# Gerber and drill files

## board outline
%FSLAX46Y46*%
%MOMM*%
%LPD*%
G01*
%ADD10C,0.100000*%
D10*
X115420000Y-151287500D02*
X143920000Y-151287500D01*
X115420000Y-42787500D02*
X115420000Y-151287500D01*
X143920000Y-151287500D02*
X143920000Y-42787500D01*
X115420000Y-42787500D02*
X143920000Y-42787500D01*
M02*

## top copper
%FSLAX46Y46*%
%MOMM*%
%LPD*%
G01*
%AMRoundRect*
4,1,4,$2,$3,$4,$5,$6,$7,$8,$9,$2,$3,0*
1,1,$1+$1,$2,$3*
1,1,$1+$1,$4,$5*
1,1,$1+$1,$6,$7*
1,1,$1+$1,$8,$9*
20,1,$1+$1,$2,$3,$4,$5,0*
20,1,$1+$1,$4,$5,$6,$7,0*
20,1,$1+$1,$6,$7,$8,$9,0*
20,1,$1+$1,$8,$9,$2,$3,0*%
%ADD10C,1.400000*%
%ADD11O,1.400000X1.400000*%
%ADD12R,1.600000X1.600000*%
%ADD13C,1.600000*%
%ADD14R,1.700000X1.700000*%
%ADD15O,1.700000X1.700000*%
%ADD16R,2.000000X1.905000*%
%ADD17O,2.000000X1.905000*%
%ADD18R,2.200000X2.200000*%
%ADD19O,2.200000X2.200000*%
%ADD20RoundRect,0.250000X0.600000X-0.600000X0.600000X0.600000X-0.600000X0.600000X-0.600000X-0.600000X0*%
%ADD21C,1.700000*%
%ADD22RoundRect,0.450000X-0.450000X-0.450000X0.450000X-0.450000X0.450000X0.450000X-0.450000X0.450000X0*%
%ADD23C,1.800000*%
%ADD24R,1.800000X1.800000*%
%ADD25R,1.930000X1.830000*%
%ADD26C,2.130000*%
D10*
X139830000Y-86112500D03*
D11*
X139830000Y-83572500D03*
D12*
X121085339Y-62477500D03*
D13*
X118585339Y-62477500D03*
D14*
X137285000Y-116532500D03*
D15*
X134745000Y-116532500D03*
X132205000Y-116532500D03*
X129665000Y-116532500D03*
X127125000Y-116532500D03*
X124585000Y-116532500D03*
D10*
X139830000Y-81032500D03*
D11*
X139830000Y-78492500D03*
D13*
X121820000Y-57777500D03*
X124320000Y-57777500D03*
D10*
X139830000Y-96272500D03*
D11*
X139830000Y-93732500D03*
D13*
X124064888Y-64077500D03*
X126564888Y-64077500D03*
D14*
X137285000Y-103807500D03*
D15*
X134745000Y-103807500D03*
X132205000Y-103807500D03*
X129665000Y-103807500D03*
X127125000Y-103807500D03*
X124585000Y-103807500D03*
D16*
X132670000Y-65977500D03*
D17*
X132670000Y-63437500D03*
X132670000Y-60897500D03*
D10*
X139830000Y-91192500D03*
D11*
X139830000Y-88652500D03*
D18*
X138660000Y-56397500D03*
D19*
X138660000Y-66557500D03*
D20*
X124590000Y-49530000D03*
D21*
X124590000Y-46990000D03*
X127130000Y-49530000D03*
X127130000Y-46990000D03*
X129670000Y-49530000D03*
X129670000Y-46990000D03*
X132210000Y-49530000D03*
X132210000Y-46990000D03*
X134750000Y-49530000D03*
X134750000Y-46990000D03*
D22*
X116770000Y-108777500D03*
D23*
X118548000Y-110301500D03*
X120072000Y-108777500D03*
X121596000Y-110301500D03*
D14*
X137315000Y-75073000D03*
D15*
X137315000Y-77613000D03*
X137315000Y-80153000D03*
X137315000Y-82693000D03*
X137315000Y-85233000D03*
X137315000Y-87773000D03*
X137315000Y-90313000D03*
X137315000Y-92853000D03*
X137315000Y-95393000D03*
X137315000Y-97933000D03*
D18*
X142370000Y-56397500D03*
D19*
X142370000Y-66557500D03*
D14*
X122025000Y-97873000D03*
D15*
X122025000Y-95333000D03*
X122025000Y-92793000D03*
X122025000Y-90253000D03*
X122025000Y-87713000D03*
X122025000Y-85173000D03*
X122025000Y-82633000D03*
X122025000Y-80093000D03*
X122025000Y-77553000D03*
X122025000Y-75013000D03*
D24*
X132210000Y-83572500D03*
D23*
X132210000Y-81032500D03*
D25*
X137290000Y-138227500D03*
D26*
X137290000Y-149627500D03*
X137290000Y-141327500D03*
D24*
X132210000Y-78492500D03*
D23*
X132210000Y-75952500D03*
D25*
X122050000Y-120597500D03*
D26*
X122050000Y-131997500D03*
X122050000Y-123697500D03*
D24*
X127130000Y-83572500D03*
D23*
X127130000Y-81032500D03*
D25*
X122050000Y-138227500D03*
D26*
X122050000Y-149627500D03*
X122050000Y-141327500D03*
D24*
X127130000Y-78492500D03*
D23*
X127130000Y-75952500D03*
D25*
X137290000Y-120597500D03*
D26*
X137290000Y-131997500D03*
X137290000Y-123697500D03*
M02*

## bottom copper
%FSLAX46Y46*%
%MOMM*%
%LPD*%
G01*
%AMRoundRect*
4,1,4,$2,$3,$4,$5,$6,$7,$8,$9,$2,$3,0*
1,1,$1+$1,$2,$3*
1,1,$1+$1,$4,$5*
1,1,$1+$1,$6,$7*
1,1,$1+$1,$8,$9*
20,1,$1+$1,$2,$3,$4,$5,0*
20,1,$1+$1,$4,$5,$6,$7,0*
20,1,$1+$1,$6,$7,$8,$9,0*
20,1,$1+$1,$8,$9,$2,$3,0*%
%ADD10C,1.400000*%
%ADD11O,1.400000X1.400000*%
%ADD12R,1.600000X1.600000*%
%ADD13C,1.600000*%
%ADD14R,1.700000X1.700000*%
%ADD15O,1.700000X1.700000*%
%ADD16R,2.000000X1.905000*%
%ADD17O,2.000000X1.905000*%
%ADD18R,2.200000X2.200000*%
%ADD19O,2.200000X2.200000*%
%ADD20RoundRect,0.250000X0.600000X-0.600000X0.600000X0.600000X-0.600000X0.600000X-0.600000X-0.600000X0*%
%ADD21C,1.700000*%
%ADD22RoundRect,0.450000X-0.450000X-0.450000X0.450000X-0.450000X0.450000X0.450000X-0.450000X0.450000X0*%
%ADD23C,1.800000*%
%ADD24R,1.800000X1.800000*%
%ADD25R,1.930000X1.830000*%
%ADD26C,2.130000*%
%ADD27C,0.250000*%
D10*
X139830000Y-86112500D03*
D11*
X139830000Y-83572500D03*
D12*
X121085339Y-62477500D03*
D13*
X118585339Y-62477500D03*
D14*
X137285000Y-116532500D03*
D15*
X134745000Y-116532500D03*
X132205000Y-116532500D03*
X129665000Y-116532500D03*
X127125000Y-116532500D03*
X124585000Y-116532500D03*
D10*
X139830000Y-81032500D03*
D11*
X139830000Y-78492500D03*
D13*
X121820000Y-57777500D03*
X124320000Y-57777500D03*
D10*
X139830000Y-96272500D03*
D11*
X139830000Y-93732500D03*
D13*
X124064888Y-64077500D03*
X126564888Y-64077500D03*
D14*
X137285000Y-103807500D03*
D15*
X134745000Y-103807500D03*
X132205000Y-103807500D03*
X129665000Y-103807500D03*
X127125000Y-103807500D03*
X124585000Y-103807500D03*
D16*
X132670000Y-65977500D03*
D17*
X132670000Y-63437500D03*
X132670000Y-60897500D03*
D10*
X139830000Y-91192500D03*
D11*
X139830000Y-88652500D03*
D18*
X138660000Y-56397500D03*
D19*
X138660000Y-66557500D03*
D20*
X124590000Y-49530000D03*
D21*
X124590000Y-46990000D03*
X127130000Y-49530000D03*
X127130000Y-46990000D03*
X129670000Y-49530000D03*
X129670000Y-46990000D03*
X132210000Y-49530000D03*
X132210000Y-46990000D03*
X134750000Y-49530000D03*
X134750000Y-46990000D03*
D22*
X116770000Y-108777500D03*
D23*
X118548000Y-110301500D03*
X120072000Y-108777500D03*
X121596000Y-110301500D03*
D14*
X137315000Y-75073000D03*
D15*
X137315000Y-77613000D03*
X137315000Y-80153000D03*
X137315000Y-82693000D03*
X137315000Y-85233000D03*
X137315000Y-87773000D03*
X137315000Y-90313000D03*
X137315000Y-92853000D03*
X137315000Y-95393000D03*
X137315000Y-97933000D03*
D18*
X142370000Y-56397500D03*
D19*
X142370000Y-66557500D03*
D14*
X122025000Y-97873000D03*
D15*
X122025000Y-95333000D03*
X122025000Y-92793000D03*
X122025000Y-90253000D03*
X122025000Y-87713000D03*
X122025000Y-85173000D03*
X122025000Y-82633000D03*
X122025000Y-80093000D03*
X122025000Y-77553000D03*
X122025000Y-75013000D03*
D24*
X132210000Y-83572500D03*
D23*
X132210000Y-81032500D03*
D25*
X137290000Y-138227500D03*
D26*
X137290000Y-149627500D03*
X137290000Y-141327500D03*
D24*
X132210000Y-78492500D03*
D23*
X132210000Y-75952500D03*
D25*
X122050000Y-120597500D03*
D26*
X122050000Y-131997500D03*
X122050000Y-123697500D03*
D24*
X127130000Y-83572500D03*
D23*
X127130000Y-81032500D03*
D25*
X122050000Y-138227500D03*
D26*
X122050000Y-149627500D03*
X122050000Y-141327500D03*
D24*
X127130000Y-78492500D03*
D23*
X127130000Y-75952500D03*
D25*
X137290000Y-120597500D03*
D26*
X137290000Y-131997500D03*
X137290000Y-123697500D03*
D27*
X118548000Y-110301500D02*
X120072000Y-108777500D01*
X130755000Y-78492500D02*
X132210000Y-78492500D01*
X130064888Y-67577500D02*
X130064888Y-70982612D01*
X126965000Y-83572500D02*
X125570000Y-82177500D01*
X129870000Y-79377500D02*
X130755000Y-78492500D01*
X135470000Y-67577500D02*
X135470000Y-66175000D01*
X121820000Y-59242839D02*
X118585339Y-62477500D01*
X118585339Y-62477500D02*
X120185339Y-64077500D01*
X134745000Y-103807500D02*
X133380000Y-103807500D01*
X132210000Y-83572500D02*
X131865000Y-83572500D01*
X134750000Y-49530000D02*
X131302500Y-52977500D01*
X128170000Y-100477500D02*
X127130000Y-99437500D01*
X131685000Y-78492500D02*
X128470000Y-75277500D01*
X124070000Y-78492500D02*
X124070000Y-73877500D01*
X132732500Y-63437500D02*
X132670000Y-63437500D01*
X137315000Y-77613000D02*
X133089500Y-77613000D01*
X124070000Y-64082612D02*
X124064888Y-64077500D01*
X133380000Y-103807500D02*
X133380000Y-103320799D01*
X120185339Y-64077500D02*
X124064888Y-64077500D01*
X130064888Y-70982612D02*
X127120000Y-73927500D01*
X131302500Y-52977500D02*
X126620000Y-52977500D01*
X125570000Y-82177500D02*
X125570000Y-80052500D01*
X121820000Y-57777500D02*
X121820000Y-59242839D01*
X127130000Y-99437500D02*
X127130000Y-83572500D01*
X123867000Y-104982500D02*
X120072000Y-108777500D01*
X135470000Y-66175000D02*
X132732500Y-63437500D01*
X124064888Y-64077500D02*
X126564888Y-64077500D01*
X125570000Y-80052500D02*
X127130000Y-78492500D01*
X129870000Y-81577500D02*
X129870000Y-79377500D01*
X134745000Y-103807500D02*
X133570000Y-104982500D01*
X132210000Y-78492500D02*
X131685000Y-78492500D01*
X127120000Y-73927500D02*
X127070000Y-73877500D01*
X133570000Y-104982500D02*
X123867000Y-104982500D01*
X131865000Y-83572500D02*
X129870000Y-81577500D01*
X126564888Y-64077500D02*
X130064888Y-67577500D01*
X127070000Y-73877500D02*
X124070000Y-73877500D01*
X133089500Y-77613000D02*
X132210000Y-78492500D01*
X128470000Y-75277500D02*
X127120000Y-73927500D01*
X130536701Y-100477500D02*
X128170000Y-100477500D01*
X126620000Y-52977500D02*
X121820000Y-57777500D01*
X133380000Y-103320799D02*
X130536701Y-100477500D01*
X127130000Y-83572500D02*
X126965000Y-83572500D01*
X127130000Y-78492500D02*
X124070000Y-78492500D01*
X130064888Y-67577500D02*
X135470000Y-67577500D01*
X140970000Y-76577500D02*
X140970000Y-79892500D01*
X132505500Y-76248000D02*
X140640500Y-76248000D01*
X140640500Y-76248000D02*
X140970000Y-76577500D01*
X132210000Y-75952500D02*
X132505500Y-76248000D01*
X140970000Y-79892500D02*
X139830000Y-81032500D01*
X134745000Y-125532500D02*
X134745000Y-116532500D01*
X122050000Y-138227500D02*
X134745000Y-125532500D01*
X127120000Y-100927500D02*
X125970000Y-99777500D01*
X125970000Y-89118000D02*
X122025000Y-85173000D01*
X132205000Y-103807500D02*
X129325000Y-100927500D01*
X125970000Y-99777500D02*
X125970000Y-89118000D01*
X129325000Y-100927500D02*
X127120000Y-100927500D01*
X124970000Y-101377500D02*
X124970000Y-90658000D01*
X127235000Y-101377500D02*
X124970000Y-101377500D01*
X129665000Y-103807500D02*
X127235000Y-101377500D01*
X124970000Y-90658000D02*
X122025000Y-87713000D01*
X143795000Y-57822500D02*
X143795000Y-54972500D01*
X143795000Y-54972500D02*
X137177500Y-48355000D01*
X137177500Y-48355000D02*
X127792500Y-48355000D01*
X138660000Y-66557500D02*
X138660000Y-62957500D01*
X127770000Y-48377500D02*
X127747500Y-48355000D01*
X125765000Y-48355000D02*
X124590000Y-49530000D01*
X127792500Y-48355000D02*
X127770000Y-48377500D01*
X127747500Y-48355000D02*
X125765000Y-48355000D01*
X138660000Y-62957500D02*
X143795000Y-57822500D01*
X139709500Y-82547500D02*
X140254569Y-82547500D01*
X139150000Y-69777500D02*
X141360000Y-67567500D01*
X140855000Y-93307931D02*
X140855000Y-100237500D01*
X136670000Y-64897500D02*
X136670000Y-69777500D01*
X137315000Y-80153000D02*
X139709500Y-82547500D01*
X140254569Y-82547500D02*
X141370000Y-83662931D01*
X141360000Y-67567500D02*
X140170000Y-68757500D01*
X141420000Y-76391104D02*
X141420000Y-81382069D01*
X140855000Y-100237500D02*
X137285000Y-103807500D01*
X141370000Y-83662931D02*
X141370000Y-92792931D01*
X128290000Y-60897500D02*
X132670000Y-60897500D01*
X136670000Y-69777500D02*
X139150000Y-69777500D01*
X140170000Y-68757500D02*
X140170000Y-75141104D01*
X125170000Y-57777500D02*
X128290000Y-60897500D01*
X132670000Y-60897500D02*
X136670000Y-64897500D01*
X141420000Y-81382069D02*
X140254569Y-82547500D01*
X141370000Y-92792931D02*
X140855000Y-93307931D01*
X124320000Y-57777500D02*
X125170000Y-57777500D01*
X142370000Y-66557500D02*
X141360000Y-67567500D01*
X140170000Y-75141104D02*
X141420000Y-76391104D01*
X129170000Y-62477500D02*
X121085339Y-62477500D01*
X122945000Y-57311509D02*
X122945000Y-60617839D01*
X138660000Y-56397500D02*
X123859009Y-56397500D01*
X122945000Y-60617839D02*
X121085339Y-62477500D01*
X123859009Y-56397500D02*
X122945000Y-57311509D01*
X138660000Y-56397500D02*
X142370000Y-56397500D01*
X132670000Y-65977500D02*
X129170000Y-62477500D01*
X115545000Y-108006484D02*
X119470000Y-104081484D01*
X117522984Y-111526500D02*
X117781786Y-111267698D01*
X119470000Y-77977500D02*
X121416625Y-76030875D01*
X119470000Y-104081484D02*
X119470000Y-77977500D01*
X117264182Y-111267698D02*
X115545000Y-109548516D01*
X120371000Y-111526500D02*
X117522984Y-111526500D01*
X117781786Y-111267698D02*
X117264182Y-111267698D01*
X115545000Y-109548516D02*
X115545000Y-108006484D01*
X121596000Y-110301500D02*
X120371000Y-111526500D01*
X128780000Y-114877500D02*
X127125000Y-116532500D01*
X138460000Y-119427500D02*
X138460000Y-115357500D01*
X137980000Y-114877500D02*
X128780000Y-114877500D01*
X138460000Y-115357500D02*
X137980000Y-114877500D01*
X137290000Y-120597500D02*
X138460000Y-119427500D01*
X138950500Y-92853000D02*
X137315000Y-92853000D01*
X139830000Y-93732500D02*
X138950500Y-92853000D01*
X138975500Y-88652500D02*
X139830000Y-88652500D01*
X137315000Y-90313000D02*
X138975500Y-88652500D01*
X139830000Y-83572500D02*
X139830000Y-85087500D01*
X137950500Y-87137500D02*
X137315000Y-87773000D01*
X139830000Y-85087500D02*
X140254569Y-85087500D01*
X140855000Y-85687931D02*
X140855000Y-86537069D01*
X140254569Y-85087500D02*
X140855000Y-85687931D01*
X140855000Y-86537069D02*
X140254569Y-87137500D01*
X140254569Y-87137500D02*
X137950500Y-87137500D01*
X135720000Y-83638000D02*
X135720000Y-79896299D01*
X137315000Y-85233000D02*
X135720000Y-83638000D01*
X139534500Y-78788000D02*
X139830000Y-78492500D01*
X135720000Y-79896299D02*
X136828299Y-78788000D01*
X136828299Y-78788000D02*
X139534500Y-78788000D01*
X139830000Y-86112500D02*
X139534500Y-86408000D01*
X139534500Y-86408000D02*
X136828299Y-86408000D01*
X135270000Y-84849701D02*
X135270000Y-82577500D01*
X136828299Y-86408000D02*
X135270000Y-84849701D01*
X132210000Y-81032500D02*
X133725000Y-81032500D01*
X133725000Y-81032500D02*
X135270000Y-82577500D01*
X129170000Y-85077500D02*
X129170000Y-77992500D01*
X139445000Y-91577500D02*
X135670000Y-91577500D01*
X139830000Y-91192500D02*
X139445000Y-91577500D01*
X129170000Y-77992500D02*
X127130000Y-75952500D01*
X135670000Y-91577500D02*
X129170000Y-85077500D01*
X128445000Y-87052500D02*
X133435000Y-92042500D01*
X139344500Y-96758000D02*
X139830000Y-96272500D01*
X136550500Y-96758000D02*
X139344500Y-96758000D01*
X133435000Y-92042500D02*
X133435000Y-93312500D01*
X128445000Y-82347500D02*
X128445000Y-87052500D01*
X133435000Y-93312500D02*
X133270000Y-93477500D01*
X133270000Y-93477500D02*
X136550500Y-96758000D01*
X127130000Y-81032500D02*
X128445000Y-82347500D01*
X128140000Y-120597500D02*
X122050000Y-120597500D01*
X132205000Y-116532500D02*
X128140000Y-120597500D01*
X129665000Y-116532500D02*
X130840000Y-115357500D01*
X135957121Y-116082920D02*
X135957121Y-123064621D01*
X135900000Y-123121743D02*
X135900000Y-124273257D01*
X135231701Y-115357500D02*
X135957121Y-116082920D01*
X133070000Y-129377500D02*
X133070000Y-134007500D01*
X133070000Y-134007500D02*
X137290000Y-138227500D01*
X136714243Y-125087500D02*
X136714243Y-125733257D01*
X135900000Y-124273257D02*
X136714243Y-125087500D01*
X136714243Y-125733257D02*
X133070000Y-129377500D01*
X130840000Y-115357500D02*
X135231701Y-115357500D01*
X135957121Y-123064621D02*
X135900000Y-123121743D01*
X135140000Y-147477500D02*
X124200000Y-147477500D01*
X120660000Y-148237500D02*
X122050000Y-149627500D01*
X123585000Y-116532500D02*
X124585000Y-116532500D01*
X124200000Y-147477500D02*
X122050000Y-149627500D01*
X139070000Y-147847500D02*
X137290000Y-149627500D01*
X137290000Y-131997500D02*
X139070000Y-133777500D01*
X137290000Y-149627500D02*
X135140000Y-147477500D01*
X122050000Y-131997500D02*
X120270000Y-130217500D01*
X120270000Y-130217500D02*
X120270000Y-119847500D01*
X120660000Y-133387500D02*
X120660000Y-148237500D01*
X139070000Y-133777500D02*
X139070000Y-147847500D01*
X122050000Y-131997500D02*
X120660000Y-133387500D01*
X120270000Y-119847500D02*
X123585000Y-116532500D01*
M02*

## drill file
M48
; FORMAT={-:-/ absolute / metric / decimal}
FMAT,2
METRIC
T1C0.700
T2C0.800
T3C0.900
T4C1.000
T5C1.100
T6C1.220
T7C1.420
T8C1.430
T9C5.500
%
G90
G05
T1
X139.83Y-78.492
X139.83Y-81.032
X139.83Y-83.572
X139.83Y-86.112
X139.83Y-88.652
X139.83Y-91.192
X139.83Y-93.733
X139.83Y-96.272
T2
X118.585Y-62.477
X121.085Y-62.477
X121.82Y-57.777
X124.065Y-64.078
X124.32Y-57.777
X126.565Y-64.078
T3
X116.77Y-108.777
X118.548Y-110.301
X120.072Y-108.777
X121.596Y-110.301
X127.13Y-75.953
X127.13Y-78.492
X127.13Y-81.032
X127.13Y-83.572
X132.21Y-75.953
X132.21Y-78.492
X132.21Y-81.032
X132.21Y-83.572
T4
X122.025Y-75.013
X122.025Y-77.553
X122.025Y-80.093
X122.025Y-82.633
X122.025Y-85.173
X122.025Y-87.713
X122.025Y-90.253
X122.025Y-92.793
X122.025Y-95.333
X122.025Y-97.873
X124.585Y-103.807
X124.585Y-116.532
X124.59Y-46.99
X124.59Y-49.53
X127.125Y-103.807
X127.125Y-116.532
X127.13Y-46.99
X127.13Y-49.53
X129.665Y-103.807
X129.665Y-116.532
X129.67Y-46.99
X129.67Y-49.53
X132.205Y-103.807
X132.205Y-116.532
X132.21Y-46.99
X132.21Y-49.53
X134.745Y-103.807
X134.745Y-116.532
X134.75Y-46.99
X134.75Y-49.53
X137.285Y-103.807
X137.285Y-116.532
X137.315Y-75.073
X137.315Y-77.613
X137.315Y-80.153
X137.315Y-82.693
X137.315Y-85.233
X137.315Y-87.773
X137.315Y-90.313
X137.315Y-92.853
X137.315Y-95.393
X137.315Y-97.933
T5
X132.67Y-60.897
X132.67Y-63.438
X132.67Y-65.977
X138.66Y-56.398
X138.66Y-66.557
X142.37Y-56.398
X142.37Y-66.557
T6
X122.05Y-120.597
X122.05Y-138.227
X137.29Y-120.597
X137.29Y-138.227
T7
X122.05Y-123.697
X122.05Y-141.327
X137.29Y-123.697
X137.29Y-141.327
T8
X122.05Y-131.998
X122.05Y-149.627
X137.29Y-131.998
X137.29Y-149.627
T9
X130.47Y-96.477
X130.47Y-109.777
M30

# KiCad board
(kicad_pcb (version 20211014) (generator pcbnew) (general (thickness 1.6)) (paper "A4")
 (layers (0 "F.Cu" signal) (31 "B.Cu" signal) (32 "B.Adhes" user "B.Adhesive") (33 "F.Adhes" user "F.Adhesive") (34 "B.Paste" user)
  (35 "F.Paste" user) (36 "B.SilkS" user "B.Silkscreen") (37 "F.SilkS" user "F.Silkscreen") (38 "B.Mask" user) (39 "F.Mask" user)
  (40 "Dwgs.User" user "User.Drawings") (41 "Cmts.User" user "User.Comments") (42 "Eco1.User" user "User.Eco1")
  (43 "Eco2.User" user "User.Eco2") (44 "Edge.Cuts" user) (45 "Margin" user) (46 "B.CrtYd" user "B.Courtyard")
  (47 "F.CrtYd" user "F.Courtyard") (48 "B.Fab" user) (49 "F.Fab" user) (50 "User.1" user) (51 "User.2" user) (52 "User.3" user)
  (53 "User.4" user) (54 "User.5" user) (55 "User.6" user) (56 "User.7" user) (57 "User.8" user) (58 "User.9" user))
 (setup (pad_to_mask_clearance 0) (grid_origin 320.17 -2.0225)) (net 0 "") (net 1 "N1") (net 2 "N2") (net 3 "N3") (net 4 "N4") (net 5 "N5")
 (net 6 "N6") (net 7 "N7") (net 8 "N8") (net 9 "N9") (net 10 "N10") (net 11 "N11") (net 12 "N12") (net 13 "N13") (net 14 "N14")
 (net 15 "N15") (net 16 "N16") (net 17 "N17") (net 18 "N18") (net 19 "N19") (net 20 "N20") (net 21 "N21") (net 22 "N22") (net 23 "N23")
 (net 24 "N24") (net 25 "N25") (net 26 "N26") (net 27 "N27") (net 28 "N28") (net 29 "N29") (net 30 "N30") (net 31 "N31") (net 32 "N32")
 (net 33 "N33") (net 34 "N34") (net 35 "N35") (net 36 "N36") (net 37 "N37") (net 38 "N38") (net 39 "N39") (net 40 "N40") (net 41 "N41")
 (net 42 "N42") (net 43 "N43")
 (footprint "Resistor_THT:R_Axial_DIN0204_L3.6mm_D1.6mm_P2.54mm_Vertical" (layer "F.Cu") (at 139.83 86.1125 90)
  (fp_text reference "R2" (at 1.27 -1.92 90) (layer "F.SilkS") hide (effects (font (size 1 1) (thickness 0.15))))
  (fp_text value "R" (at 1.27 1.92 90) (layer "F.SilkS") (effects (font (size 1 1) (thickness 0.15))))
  (pad "1" thru_hole circle (at 0 0 90) (size 1.4 1.4) (drill 0.7) (layers *.Cu *.Mask) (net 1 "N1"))
  (pad "2" thru_hole oval (at 2.54 0 90) (size 1.4 1.4) (drill 0.7) (layers *.Cu *.Mask) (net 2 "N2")))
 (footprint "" (layer "F.Cu") (at 130.47 109.7775)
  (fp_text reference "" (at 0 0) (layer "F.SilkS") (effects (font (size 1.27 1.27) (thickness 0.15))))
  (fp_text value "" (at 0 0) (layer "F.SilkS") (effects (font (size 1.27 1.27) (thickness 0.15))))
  (pad "" np_thru_hole circle (at 0 0) (size 5.5 5.5) (drill 5.5) (layers F&B.Cu *.Mask)))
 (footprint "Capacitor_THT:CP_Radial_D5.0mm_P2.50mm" (layer "F.Cu") (at 121.085339 62.4775 180)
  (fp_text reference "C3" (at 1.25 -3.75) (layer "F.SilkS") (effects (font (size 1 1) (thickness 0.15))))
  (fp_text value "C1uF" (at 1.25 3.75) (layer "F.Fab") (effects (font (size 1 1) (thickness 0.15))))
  (pad "1" thru_hole rect (at 0 0 180) (size 1.6 1.6) (drill 0.8) (layers *.Cu *.Mask) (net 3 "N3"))
  (pad "2" thru_hole circle (at 2.5 0 180) (size 1.6 1.6) (drill 0.8) (layers *.Cu *.Mask) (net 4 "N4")))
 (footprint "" (layer "F.Cu") (at 130.47 96.4775)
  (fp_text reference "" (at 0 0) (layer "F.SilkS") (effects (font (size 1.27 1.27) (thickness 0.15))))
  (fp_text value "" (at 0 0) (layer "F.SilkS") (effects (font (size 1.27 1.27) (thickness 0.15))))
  (pad "" np_thru_hole circle (at 0 0) (size 5.5 5.5) (drill 5.5) (layers F&B.Cu *.Mask)))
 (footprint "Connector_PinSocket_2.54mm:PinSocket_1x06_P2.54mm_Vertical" (layer "F.Cu") (at 137.285 116.5325 -90)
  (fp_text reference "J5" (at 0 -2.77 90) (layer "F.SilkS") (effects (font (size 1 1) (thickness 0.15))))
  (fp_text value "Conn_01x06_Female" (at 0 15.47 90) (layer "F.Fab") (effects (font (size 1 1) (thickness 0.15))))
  (pad "1" thru_hole rect (at 0 0 270) (size 1.7 1.7) (drill 1) (layers *.Cu *.Mask) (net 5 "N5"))
  (pad "2" thru_hole oval (at 0 2.54 270) (size 1.7 1.7) (drill 1) (layers *.Cu *.Mask) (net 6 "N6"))
  (pad "3" thru_hole oval (at 0 5.08 270) (size 1.7 1.7) (drill 1) (layers *.Cu *.Mask) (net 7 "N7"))
  (pad "4" thru_hole oval (at 0 7.62 270) (size 1.7 1.7) (drill 1) (layers *.Cu *.Mask) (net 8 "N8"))
  (pad "5" thru_hole oval (at 0 10.16 270) (size 1.7 1.7) (drill 1) (layers *.Cu *.Mask) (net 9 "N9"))
  (pad "6" thru_hole oval (at 0 12.7 270) (size 1.7 1.7) (drill 1) (layers *.Cu *.Mask) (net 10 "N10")))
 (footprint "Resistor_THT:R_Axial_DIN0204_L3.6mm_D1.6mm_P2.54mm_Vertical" (layer "F.Cu") (at 139.83 81.0325 90)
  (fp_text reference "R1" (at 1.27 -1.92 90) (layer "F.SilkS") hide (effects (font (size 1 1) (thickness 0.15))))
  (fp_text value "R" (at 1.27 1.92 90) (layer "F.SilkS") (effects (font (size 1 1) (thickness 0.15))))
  (pad "1" thru_hole circle (at 0 0 90) (size 1.4 1.4) (drill 0.7) (layers *.Cu *.Mask) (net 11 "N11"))
  (pad "2" thru_hole oval (at 2.54 0 90) (size 1.4 1.4) (drill 0.7) (layers *.Cu *.Mask) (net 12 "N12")))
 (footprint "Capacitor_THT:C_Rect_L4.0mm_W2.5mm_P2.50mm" (layer "F.Cu") (at 121.82 57.7775)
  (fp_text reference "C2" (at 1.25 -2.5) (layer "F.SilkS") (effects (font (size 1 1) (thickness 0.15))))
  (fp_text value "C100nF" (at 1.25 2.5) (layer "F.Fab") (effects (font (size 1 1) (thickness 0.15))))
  (pad "1" thru_hole circle (at 0 0) (size 1.6 1.6) (drill 0.8) (layers *.Cu *.Mask) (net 4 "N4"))
  (pad "2" thru_hole circle (at 2.5 0) (size 1.6 1.6) (drill 0.8) (layers *.Cu *.Mask) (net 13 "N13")))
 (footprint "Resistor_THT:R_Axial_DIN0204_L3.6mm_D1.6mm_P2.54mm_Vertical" (layer "F.Cu") (at 139.83 96.2725 90)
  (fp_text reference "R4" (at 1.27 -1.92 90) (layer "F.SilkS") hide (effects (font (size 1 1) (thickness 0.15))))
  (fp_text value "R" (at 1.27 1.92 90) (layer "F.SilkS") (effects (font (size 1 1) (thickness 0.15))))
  (pad "1" thru_hole circle (at 0 0 90) (size 1.4 1.4) (drill 0.7) (layers *.Cu *.Mask) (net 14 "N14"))
  (pad "2" thru_hole oval (at 2.54 0 90) (size 1.4 1.4) (drill 0.7) (layers *.Cu *.Mask) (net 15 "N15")))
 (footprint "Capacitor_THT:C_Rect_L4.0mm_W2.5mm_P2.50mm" (layer "F.Cu") (at 124.064888 64.0775)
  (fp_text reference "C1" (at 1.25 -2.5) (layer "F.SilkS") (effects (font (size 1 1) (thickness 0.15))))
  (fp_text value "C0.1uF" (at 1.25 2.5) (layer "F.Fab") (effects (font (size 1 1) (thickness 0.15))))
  (pad "1" thru_hole circle (at 0 0) (size 1.6 1.6) (drill 0.8) (layers *.Cu *.Mask) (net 4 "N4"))
  (pad "2" thru_hole circle (at 2.5 0) (size 1.6 1.6) (drill 0.8) (layers *.Cu *.Mask) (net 4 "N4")))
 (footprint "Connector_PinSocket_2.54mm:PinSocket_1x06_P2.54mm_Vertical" (layer "F.Cu") (at 137.285 103.8075 -90)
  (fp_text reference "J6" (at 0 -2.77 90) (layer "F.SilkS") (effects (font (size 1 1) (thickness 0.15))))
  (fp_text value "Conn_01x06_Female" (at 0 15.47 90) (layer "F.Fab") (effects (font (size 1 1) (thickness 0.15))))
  (pad "1" thru_hole rect (at 0 0 270) (size 1.7 1.7) (drill 1) (layers *.Cu *.Mask) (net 13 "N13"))
  (pad "2" thru_hole oval (at 0 2.54 270) (size 1.7 1.7) (drill 1) (layers *.Cu *.Mask) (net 4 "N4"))
  (pad "3" thru_hole oval (at 0 5.08 270) (size 1.7 1.7) (drill 1) (layers *.Cu *.Mask) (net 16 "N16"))
  (pad "4" thru_hole oval (at 0 7.62 270) (size 1.7 1.7) (drill 1) (layers *.Cu *.Mask) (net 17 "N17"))
  (pad "5" thru_hole oval (at 0 10.16 270) (size 1.7 1.7) (drill 1) (layers *.Cu *.Mask) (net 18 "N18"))
  (pad "6" thru_hole oval (at 0 12.7 270) (size 1.7 1.7) (drill 1) (layers *.Cu *.Mask) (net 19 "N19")))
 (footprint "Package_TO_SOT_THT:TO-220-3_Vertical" (layer "F.Cu") (at 132.67 65.9775 90)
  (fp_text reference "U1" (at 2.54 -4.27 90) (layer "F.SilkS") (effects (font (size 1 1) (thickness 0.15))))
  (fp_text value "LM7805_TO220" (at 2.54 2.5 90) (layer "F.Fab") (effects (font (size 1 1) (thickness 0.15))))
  (pad "1" thru_hole rect (at 0 0 90) (size 1.905 2) (drill 1.1) (layers *.Cu *.Mask) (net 3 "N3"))
  (pad "2" thru_hole oval (at 2.54 0 90) (size 1.905 2) (drill 1.1) (layers *.Cu *.Mask) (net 4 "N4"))
  (pad "3" thru_hole oval (at 5.08 0 90) (size 1.905 2) (drill 1.1) (layers *.Cu *.Mask) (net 13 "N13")))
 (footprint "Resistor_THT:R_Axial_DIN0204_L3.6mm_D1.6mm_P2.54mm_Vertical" (layer "F.Cu") (at 139.83 91.1925 90)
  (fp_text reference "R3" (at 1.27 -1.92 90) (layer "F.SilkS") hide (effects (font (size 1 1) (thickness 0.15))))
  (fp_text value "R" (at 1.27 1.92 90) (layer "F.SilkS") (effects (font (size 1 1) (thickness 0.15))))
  (pad "1" thru_hole circle (at 0 0 90) (size 1.4 1.4) (drill 0.7) (layers *.Cu *.Mask) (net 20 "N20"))
  (pad "2" thru_hole oval (at 2.54 0 90) (size 1.4 1.4) (drill 0.7) (layers *.Cu *.Mask) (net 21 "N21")))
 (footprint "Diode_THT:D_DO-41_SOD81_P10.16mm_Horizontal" (layer "F.Cu") (at 138.66 56.3975 -90)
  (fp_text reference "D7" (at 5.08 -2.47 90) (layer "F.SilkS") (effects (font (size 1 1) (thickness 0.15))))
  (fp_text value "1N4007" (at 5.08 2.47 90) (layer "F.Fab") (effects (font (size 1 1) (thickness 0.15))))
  (pad "1" thru_hole rect (at 0 0 270) (size 2.2 2.2) (drill 1.1) (layers *.Cu *.Mask) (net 3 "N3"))
  (pad "2" thru_hole oval (at 10.16 0 270) (size 2.2 2.2) (drill 1.1) (layers *.Cu *.Mask) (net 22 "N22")))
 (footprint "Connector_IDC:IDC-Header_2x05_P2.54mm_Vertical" (layer "F.Cu") (at 124.59 49.53 90)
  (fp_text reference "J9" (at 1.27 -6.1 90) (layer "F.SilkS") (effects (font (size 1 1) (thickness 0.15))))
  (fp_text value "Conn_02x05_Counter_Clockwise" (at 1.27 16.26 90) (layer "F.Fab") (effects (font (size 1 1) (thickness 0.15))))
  (pad "1" thru_hole roundrect (at 0 0 90) (size 1.7 1.7) (drill 1) (layers *.Cu *.Mask) (roundrect_rratio 0.147059) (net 22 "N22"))
  (pad "2" thru_hole circle (at 2.54 0 90) (size 1.7 1.7) (drill 1) (layers *.Cu *.Mask) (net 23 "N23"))
  (pad "3" thru_hole circle (at 0 2.54 90) (size 1.7 1.7) (drill 1) (layers *.Cu *.Mask) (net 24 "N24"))
  (pad "4" thru_hole circle (at 2.54 2.54 90) (size 1.7 1.7) (drill 1) (layers *.Cu *.Mask) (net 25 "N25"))
  (pad "5" thru_hole circle (at 0 5.08 90) (size 1.7 1.7) (drill 1) (layers *.Cu *.Mask) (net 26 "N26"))
  (pad "6" thru_hole circle (at 2.54 5.08 90) (size 1.7 1.7) (drill 1) (layers *.Cu *.Mask) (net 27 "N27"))
  (pad "7" thru_hole circle (at 0 7.62 90) (size 1.7 1.7) (drill 1) (layers *.Cu *.Mask) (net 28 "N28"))
  (pad "8" thru_hole circle (at 2.54 7.62 90) (size 1.7 1.7) (drill 1) (layers *.Cu *.Mask) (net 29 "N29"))
  (pad "9" thru_hole circle (at 0 10.16 90) (size 1.7 1.7) (drill 1) (layers *.Cu *.Mask) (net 4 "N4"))
  (pad "10" thru_hole circle (at 2.54 10.16 90) (size 1.7 1.7) (drill 1) (layers *.Cu *.Mask) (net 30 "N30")))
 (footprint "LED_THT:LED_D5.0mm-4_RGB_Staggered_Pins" (layer "F.Cu") (at 116.77 108.7775)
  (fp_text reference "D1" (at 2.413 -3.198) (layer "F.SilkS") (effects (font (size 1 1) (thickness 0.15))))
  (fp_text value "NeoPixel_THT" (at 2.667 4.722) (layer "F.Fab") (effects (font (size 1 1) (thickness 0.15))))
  (pad "1" thru_hole roundrect (at 0 0) (size 1.8 1.8) (drill 0.9) (layers *.Cu *.Mask) (roundrect_rratio 0.25) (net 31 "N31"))
  (pad "2" thru_hole circle (at 1.778 1.524) (size 1.8 1.8) (drill 0.9) (layers *.Cu *.Mask) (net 4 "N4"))
  (pad "3" thru_hole circle (at 3.302 0) (size 1.8 1.8) (drill 0.9) (layers *.Cu *.Mask) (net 4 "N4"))
  (pad "4" thru_hole circle (at 4.826 1.524) (size 1.8 1.8) (drill 0.9) (layers *.Cu *.Mask) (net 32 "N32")))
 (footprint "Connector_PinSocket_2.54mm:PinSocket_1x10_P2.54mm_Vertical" (layer "F.Cu") (at 137.315 75.073)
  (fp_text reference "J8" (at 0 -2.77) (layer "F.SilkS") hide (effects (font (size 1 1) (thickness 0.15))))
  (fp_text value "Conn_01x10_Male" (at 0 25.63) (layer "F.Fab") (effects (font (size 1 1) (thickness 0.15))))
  (pad "1" thru_hole rect (at 0 0) (size 1.7 1.7) (drill 1) (layers *.Cu *.Mask) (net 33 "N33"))
  (pad "2" thru_hole oval (at 0 2.54) (size 1.7 1.7) (drill 1) (layers *.Cu *.Mask) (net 4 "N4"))
  (pad "3" thru_hole oval (at 0 5.08) (size 1.7 1.7) (drill 1) (layers *.Cu *.Mask) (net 13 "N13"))
  (pad "4" thru_hole oval (at 0 7.62) (size 1.7 1.7) (drill 1) (layers *.Cu *.Mask) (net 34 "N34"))
  (pad "5" thru_hole oval (at 0 10.16) (size 1.7 1.7) (drill 1) (layers *.Cu *.Mask) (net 12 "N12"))
  (pad "6" thru_hole oval (at 0 12.7) (size 1.7 1.7) (drill 1) (layers *.Cu *.Mask) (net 2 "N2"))
  (pad "7" thru_hole oval (at 0 15.24) (size 1.7 1.7) (drill 1) (layers *.Cu *.Mask) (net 21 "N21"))
  (pad "8" thru_hole oval (at 0 17.78) (size 1.7 1.7) (drill 1) (layers *.Cu *.Mask) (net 15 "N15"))
  (pad "9" thru_hole oval (at 0 20.32) (size 1.7 1.7) (drill 1) (layers *.Cu *.Mask) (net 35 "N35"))
  (pad "10" thru_hole oval (at 0 22.86) (size 1.7 1.7) (drill 1) (layers *.Cu *.Mask) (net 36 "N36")))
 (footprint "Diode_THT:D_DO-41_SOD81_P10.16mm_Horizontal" (layer "F.Cu") (at 142.37 56.3975 -90)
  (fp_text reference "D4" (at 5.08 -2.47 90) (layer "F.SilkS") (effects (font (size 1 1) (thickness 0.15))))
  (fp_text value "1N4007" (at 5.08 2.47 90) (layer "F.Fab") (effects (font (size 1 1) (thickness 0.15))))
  (pad "1" thru_hole rect (at 0 0 270) (size 2.2 2.2) (drill 1.1) (layers *.Cu *.Mask) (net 3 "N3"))
  (pad "2" thru_hole oval (at 10.16 0 270) (size 2.2 2.2) (drill 1.1) (layers *.Cu *.Mask) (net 13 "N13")))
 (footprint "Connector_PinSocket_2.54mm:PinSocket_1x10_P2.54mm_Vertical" (layer "F.Cu") (at 122.025 97.873 180)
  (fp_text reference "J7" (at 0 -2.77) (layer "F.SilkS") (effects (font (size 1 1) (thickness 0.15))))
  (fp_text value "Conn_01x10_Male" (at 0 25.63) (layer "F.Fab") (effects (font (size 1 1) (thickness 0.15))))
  (pad "1" thru_hole rect (at 0 0 180) (size 1.7 1.7) (drill 1) (layers *.Cu *.Mask) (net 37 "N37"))
  (pad "2" thru_hole oval (at 0 2.54 180) (size 1.7 1.7) (drill 1) (layers *.Cu *.Mask) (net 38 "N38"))
  (pad "3" thru_hole oval (at 0 5.08 180) (size 1.7 1.7) (drill 1) (layers *.Cu *.Mask) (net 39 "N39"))
  (pad "4" thru_hole oval (at 0 7.62 180) (size 1.7 1.7) (drill 1) (layers *.Cu *.Mask) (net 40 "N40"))
  (pad "5" thru_hole oval (at 0 10.16 180) (size 1.7 1.7) (drill 1) (layers *.Cu *.Mask) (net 17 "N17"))
  (pad "6" thru_hole oval (at 0 12.7 180) (size 1.7 1.7) (drill 1) (layers *.Cu *.Mask) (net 16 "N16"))
  (pad "7" thru_hole oval (at 0 15.24 180) (size 1.7 1.7) (drill 1) (layers *.Cu *.Mask) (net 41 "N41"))
  (pad "8" thru_hole oval (at 0 17.78 180) (size 1.7 1.7) (drill 1) (layers *.Cu *.Mask) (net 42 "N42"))
  (pad "9" thru_hole oval (at 0 20.32 180) (size 1.7 1.7) (drill 1) (layers *.Cu *.Mask) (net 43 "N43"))
  (pad "10" thru_hole oval (at 0 22.86 180) (size 1.7 1.7) (drill 1) (layers *.Cu *.Mask) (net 32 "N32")))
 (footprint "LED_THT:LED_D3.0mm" (layer "B.Cu") (at 132.21 83.5725 90)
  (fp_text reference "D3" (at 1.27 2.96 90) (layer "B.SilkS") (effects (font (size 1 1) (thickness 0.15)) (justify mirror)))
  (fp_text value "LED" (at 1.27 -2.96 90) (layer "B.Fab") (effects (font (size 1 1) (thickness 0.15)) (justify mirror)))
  (pad "1" thru_hole rect (at 0 0 90) (size 1.8 1.8) (drill 0.9) (layers *.Cu *.Mask) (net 4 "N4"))
  (pad "2" thru_hole circle (at 2.54 0 90) (size 1.8 1.8) (drill 0.9) (layers *.Cu *.Mask) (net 1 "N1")))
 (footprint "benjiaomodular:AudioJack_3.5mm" (layer "B.Cu") (at 137.29 138.2275 180)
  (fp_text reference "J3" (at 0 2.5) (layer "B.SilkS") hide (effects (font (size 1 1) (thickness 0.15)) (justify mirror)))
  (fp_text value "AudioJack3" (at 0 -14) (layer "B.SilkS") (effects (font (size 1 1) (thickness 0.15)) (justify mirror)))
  (pad "S" thru_hole rect locked (at 0 0) (size 1.93 1.83) (drill 1.22) (layers *.Cu *.Mask) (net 8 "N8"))
  (pad "T" thru_hole circle locked (at 0 -11.4) (size 2.13 2.13) (drill 1.43) (layers *.Cu *.Mask) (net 10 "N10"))
  (pad "TN" thru_hole circle locked (at 0 -3.1) (size 2.13 2.13) (drill 1.42) (layers *.Cu *.Mask)))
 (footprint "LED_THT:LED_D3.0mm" (layer "B.Cu") (at 132.21 78.4925 90)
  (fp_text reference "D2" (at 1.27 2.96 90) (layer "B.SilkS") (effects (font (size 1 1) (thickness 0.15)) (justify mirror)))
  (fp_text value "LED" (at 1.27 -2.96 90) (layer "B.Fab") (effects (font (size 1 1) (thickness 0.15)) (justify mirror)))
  (pad "1" thru_hole rect (at 0 0 90) (size 1.8 1.8) (drill 0.9) (layers *.Cu *.Mask) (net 4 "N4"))
  (pad "2" thru_hole circle (at 2.54 0 90) (size 1.8 1.8) (drill 0.9) (layers *.Cu *.Mask) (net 11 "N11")))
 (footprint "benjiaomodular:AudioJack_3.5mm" (layer "B.Cu") (at 122.05 120.5975 180)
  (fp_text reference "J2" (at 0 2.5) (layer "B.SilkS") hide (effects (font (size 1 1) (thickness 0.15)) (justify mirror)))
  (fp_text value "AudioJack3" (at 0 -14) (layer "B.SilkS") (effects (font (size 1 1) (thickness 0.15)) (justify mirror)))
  (pad "S" thru_hole rect locked (at 0 0) (size 1.93 1.83) (drill 1.22) (layers *.Cu *.Mask) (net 7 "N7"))
  (pad "T" thru_hole circle locked (at 0 -11.4) (size 2.13 2.13) (drill 1.43) (layers *.Cu *.Mask) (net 10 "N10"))
  (pad "TN" thru_hole circle locked (at 0 -3.1) (size 2.13 2.13) (drill 1.42) (layers *.Cu *.Mask)))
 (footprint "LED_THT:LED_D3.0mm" (layer "B.Cu") (at 127.13 83.5725 90)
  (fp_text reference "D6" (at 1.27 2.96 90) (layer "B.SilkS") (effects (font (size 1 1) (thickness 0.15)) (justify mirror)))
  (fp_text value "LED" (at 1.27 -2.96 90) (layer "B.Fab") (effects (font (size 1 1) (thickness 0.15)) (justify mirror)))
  (pad "1" thru_hole rect (at 0 0 90) (size 1.8 1.8) (drill 0.9) (layers *.Cu *.Mask) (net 4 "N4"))
  (pad "2" thru_hole circle (at 2.54 0 90) (size 1.8 1.8) (drill 0.9) (layers *.Cu *.Mask) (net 14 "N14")))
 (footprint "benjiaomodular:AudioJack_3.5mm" (layer "B.Cu") (at 122.05 138.2275 180)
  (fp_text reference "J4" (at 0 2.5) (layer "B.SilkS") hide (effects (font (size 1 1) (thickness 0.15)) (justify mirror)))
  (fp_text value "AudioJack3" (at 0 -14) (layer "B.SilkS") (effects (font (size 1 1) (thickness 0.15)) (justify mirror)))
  (pad "S" thru_hole rect locked (at 0 0) (size 1.93 1.83) (drill 1.22) (layers *.Cu *.Mask) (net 6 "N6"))
  (pad "T" thru_hole circle locked (at 0 -11.4) (size 2.13 2.13) (drill 1.43) (layers *.Cu *.Mask) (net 10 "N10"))
  (pad "TN" thru_hole circle locked (at 0 -3.1) (size 2.13 2.13) (drill 1.42) (layers *.Cu *.Mask)))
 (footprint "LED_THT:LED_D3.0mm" (layer "B.Cu") (at 127.13 78.4925 90)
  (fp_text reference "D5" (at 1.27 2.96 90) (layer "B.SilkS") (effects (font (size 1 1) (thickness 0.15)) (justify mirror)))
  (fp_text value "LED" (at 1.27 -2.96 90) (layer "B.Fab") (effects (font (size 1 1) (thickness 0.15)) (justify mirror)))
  (pad "1" thru_hole rect (at 0 0 90) (size 1.8 1.8) (drill 0.9) (layers *.Cu *.Mask) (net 4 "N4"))
  (pad "2" thru_hole circle (at 2.54 0 90) (size 1.8 1.8) (drill 0.9) (layers *.Cu *.Mask) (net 20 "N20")))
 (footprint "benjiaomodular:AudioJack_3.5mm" (layer "B.Cu") (at 137.29 120.5975 180)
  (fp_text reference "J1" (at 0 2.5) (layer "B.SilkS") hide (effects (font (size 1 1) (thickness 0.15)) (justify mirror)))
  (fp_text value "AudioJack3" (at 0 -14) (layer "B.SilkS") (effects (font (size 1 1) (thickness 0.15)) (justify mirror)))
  (pad "S" thru_hole rect locked (at 0 0) (size 1.93 1.83) (drill 1.22) (layers *.Cu *.Mask) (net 9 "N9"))
  (pad "T" thru_hole circle locked (at 0 -11.4) (size 2.13 2.13) (drill 1.43) (layers *.Cu *.Mask) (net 10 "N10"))
  (pad "TN" thru_hole circle locked (at 0 -3.1) (size 2.13 2.13) (drill 1.42) (layers *.Cu *.Mask)))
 (gr_line (start 115.42 151.2875) (end 143.92 151.2875) (layer "Edge.Cuts") (width 0.1))
 (gr_line (start 115.42 42.7875) (end 115.42 151.2875) (layer "Edge.Cuts") (width 0.1))
 (gr_line (start 143.92 151.2875) (end 143.92 42.7875) (layer "Edge.Cuts") (width 0.1))
 (gr_line (start 115.42 42.7875) (end 143.92 42.7875) (layer "Edge.Cuts") (width 0.1))
 (segment (start 118.548 110.3015) (end 120.072 108.7775) (width 0.25) (layer "B.Cu") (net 4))
 (segment (start 130.755 78.4925) (end 132.21 78.4925) (width 0.25) (layer "B.Cu") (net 4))
 (segment (start 130.064888 67.5775) (end 130.064888 70.982612) (width 0.25) (layer "B.Cu") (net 4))
 (segment (start 126.965 83.5725) (end 125.57 82.1775) (width 0.25) (layer "B.Cu") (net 4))
 (segment (start 129.87 79.3775) (end 130.755 78.4925) (width 0.25) (layer "B.Cu") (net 4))
 (segment (start 135.47 67.5775) (end 135.47 66.175) (width 0.25) (layer "B.Cu") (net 4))
 (segment (start 121.82 59.242839) (end 118.585339 62.4775) (width 0.25) (layer "B.Cu") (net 4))
 (segment (start 118.585339 62.4775) (end 120.185339 64.0775) (width 0.25) (layer "B.Cu") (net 4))
 (segment (start 134.745 103.8075) (end 133.38 103.8075) (width 0.25) (layer "B.Cu") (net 4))
 (segment (start 132.21 83.5725) (end 131.865 83.5725) (width 0.25) (layer "B.Cu") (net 4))
 (segment (start 134.75 49.53) (end 131.3025 52.9775) (width 0.25) (layer "B.Cu") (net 4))
 (segment (start 128.17 100.4775) (end 127.13 99.4375) (width 0.25) (layer "B.Cu") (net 4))
 (segment (start 131.685 78.4925) (end 128.47 75.2775) (width 0.25) (layer "B.Cu") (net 4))
 (segment (start 124.07 78.4925) (end 124.07 73.8775) (width 0.25) (layer "B.Cu") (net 4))
 (segment (start 132.7325 63.4375) (end 132.67 63.4375) (width 0.25) (layer "B.Cu") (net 4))
 (segment (start 137.315 77.613) (end 133.0895 77.613) (width 0.25) (layer "B.Cu") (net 4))
 (segment (start 124.07 64.082612) (end 124.064888 64.0775) (width 0.25) (layer "B.Cu") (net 4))
 (segment (start 133.38 103.8075) (end 133.38 103.320799) (width 0.25) (layer "B.Cu") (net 4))
 (segment (start 120.185339 64.0775) (end 124.064888 64.0775) (width 0.25) (layer "B.Cu") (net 4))
 (segment (start 130.064888 70.982612) (end 127.12 73.9275) (width 0.25) (layer "B.Cu") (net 4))
 (segment (start 131.3025 52.9775) (end 126.62 52.9775) (width 0.25) (layer "B.Cu") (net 4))
 (segment (start 125.57 82.1775) (end 125.57 80.0525) (width 0.25) (layer "B.Cu") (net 4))
 (segment (start 121.82 57.7775) (end 121.82 59.242839) (width 0.25) (layer "B.Cu") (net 4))
 (segment (start 127.13 99.4375) (end 127.13 83.5725) (width 0.25) (layer "B.Cu") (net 4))
 (segment (start 123.867 104.9825) (end 120.072 108.7775) (width 0.25) (layer "B.Cu") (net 4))
 (segment (start 135.47 66.175) (end 132.7325 63.4375) (width 0.25) (layer "B.Cu") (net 4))
 (segment (start 124.064888 64.0775) (end 126.564888 64.0775) (width 0.25) (layer "B.Cu") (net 4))
 (segment (start 125.57 80.0525) (end 127.13 78.4925) (width 0.25) (layer "B.Cu") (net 4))
 (segment (start 129.87 81.5775) (end 129.87 79.3775) (width 0.25) (layer "B.Cu") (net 4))
 (segment (start 134.745 103.8075) (end 133.57 104.9825) (width 0.25) (layer "B.Cu") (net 4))
 (segment (start 132.21 78.4925) (end 131.685 78.4925) (width 0.25) (layer "B.Cu") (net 4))
 (segment (start 127.12 73.9275) (end 127.07 73.8775) (width 0.25) (layer "B.Cu") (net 4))
 (segment (start 133.57 104.9825) (end 123.867 104.9825) (width 0.25) (layer "B.Cu") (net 4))
 (segment (start 131.865 83.5725) (end 129.87 81.5775) (width 0.25) (layer "B.Cu") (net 4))
 (segment (start 126.564888 64.0775) (end 130.064888 67.5775) (width 0.25) (layer "B.Cu") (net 4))
 (segment (start 127.07 73.8775) (end 124.07 73.8775) (width 0.25) (layer "B.Cu") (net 4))
 (segment (start 133.0895 77.613) (end 132.21 78.4925) (width 0.25) (layer "B.Cu") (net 4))
 (segment (start 128.47 75.2775) (end 127.12 73.9275) (width 0.25) (layer "B.Cu") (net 4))
 (segment (start 130.536701 100.4775) (end 128.17 100.4775) (width 0.25) (layer "B.Cu") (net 4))
 (segment (start 126.62 52.9775) (end 121.82 57.7775) (width 0.25) (layer "B.Cu") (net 4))
 (segment (start 133.38 103.320799) (end 130.536701 100.4775) (width 0.25) (layer "B.Cu") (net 4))
 (segment (start 127.13 83.5725) (end 126.965 83.5725) (width 0.25) (layer "B.Cu") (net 4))
 (segment (start 127.13 78.4925) (end 124.07 78.4925) (width 0.25) (layer "B.Cu") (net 4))
 (segment (start 130.064888 67.5775) (end 135.47 67.5775) (width 0.25) (layer "B.Cu") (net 4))
 (segment (start 140.97 76.5775) (end 140.97 79.8925) (width 0.25) (layer "B.Cu") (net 11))
 (segment (start 132.5055 76.248) (end 140.6405 76.248) (width 0.25) (layer "B.Cu") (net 11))
 (segment (start 140.6405 76.248) (end 140.97 76.5775) (width 0.25) (layer "B.Cu") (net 11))
 (segment (start 132.21 75.9525) (end 132.5055 76.248) (width 0.25) (layer "B.Cu") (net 11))
 (segment (start 140.97 79.8925) (end 139.83 81.0325) (width 0.25) (layer "B.Cu") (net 11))
 (segment (start 134.745 125.5325) (end 134.745 116.5325) (width 0.25) (layer "B.Cu") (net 6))
 (segment (start 122.05 138.2275) (end 134.745 125.5325) (width 0.25) (layer "B.Cu") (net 6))
 (segment (start 127.12 100.9275) (end 125.97 99.7775) (width 0.25) (layer "B.Cu") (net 16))
 (segment (start 125.97 89.118) (end 122.025 85.173) (width 0.25) (layer "B.Cu") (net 16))
 (segment (start 132.205 103.8075) (end 129.325 100.9275) (width 0.25) (layer "B.Cu") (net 16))
 (segment (start 125.97 99.7775) (end 125.97 89.118) (width 0.25) (layer "B.Cu") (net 16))
 (segment (start 129.325 100.9275) (end 127.12 100.9275) (width 0.25) (layer "B.Cu") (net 16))
 (segment (start 124.97 101.3775) (end 124.97 90.658) (width 0.25) (layer "B.Cu") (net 17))
 (segment (start 127.235 101.3775) (end 124.97 101.3775) (width 0.25) (layer "B.Cu") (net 17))
 (segment (start 129.665 103.8075) (end 127.235 101.3775) (width 0.25) (layer "B.Cu") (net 17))
 (segment (start 124.97 90.658) (end 122.025 87.713) (width 0.25) (layer "B.Cu") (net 17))
 (segment (start 143.795 57.8225) (end 143.795 54.9725) (width 0.25) (layer "B.Cu") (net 22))
 (segment (start 143.795 54.9725) (end 137.1775 48.355) (width 0.25) (layer "B.Cu") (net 22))
 (segment (start 137.1775 48.355) (end 127.7925 48.355) (width 0.25) (layer "B.Cu") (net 22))
 (segment (start 138.66 66.5575) (end 138.66 62.9575) (width 0.25) (layer "B.Cu") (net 22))
 (segment (start 127.77 48.3775) (end 127.7475 48.355) (width 0.25) (layer "B.Cu") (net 22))
 (segment (start 125.765 48.355) (end 124.59 49.53) (width 0.25) (layer "B.Cu") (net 22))
 (segment (start 127.7925 48.355) (end 127.77 48.3775) (width 0.25) (layer "B.Cu") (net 22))
 (segment (start 127.7475 48.355) (end 125.765 48.355) (width 0.25) (layer "B.Cu") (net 22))
 (segment (start 138.66 62.9575) (end 143.795 57.8225) (width 0.25) (layer "B.Cu") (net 22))
 (segment (start 139.7095 82.5475) (end 140.254569 82.5475) (width 0.25) (layer "B.Cu") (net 13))
 (segment (start 139.15 69.7775) (end 141.36 67.5675) (width 0.25) (layer "B.Cu") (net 13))
 (segment (start 140.855 93.307931) (end 140.855 100.2375) (width 0.25) (layer "B.Cu") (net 13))
 (segment (start 136.67 64.8975) (end 136.67 69.7775) (width 0.25) (layer "B.Cu") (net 13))
 (segment (start 137.315 80.153) (end 139.7095 82.5475) (width 0.25) (layer "B.Cu") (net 13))
 (segment (start 140.254569 82.5475) (end 141.37 83.662931) (width 0.25) (layer "B.Cu") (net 13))
 (segment (start 141.36 67.5675) (end 140.17 68.7575) (width 0.25) (layer "B.Cu") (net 13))
 (segment (start 141.42 76.391104) (end 141.42 81.382069) (width 0.25) (layer "B.Cu") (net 13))
 (segment (start 140.855 100.2375) (end 137.285 103.8075) (width 0.25) (layer "B.Cu") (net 13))
 (segment (start 141.37 83.662931) (end 141.37 92.792931) (width 0.25) (layer "B.Cu") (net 13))
 (segment (start 128.29 60.8975) (end 132.67 60.8975) (width 0.25) (layer "B.Cu") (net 13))
 (segment (start 136.67 69.7775) (end 139.15 69.7775) (width 0.25) (layer "B.Cu") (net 13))
 (segment (start 140.17 68.7575) (end 140.17 75.141104) (width 0.25) (layer "B.Cu") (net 13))
 (segment (start 125.17 57.7775) (end 128.29 60.8975) (width 0.25) (layer "B.Cu") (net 13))
 (segment (start 132.67 60.8975) (end 136.67 64.8975) (width 0.25) (layer "B.Cu") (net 13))
 (segment (start 141.42 81.382069) (end 140.254569 82.5475) (width 0.25) (layer "B.Cu") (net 13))
 (segment (start 141.37 92.792931) (end 140.855 93.307931) (width 0.25) (layer "B.Cu") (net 13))
 (segment (start 124.32 57.7775) (end 125.17 57.7775) (width 0.25) (layer "B.Cu") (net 13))
 (segment (start 142.37 66.5575) (end 141.36 67.5675) (width 0.25) (layer "B.Cu") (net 13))
 (segment (start 140.17 75.141104) (end 141.42 76.391104) (width 0.25) (layer "B.Cu") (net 13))
 (segment (start 129.17 62.4775) (end 121.085339 62.4775) (width 0.25) (layer "B.Cu") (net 3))
 (segment (start 122.945 57.311509) (end 122.945 60.617839) (width 0.25) (layer "B.Cu") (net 3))
 (segment (start 138.66 56.3975) (end 123.859009 56.3975) (width 0.25) (layer "B.Cu") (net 3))
 (segment (start 122.945 60.617839) (end 121.085339 62.4775) (width 0.25) (layer "B.Cu") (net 3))
 (segment (start 123.859009 56.3975) (end 122.945 57.311509) (width 0.25) (layer "B.Cu") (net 3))
 (segment (start 138.66 56.3975) (end 142.37 56.3975) (width 0.25) (layer "B.Cu") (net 3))
 (segment (start 132.67 65.9775) (end 129.17 62.4775) (width 0.25) (layer "B.Cu") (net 3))
 (segment (start 115.545 108.006484) (end 119.47 104.081484) (width 0.25) (layer "B.Cu") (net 32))
 (segment (start 117.522984 111.5265) (end 117.781786 111.267698) (width 0.25) (layer "B.Cu") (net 32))
 (segment (start 119.47 77.9775) (end 121.416625 76.030875) (width 0.25) (layer "B.Cu") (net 32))
 (segment (start 119.47 104.081484) (end 119.47 77.9775) (width 0.25) (layer "B.Cu") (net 32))
 (segment (start 117.264182 111.267698) (end 115.545 109.548516) (width 0.25) (layer "B.Cu") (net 32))
 (segment (start 120.371 111.5265) (end 117.522984 111.5265) (width 0.25) (layer "B.Cu") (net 32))
 (segment (start 117.781786 111.267698) (end 117.264182 111.267698) (width 0.25) (layer "B.Cu") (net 32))
 (segment (start 115.545 109.548516) (end 115.545 108.006484) (width 0.25) (layer "B.Cu") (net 32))
 (segment (start 121.596 110.3015) (end 120.371 111.5265) (width 0.25) (layer "B.Cu") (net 32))
 (segment (start 128.78 114.8775) (end 127.125 116.5325) (width 0.25) (layer "B.Cu") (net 9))
 (segment (start 138.46 119.4275) (end 138.46 115.3575) (width 0.25) (layer "B.Cu") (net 9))
 (segment (start 137.98 114.8775) (end 128.78 114.8775) (width 0.25) (layer "B.Cu") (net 9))
 (segment (start 138.46 115.3575) (end 137.98 114.8775) (width 0.25) (layer "B.Cu") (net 9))
 (segment (start 137.29 120.5975) (end 138.46 119.4275) (width 0.25) (layer "B.Cu") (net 9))
 (segment (start 138.9505 92.853) (end 137.315 92.853) (width 0.25) (layer "B.Cu") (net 15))
 (segment (start 139.83 93.7325) (end 138.9505 92.853) (width 0.25) (layer "B.Cu") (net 15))
 (segment (start 138.9755 88.6525) (end 139.83 88.6525) (width 0.25) (layer "B.Cu") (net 21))
 (segment (start 137.315 90.313) (end 138.9755 88.6525) (width 0.25) (layer "B.Cu") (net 21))
 (segment (start 139.83 83.5725) (end 139.83 85.0875) (width 0.25) (layer "B.Cu") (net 2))
 (segment (start 137.9505 87.1375) (end 137.315 87.773) (width 0.25) (layer "B.Cu") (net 2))
 (segment (start 139.83 85.0875) (end 140.254569 85.0875) (width 0.25) (layer "B.Cu") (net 2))
 (segment (start 140.855 85.687931) (end 140.855 86.537069) (width 0.25) (layer "B.Cu") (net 2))
 (segment (start 140.254569 85.0875) (end 140.855 85.687931) (width 0.25) (layer "B.Cu") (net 2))
 (segment (start 140.855 86.537069) (end 140.254569 87.1375) (width 0.25) (layer "B.Cu") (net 2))
 (segment (start 140.254569 87.1375) (end 137.9505 87.1375) (width 0.25) (layer "B.Cu") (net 2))
 (segment (start 135.72 83.638) (end 135.72 79.896299) (width 0.25) (layer "B.Cu") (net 12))
 (segment (start 137.315 85.233) (end 135.72 83.638) (width 0.25) (layer "B.Cu") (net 12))
 (segment (start 139.5345 78.788) (end 139.83 78.4925) (width 0.25) (layer "B.Cu") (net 12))
 (segment (start 135.72 79.896299) (end 136.828299 78.788) (width 0.25) (layer "B.Cu") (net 12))
 (segment (start 136.828299 78.788) (end 139.5345 78.788) (width 0.25) (layer "B.Cu") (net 12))
 (segment (start 139.83 86.1125) (end 139.5345 86.408) (width 0.25) (layer "B.Cu") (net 1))
 (segment (start 139.5345 86.408) (end 136.828299 86.408) (width 0.25) (layer "B.Cu") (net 1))
 (segment (start 135.27 84.849701) (end 135.27 82.5775) (width 0.25) (layer "B.Cu") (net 1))
 (segment (start 136.828299 86.408) (end 135.27 84.849701) (width 0.25) (layer "B.Cu") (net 1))
 (segment (start 132.21 81.0325) (end 133.725 81.0325) (width 0.25) (layer "B.Cu") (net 1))
 (segment (start 133.725 81.0325) (end 135.27 82.5775) (width 0.25) (layer "B.Cu") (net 1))
 (segment (start 129.17 85.0775) (end 129.17 77.9925) (width 0.25) (layer "B.Cu") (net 20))
 (segment (start 139.445 91.5775) (end 135.67 91.5775) (width 0.25) (layer "B.Cu") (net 20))
 (segment (start 139.83 91.1925) (end 139.445 91.5775) (width 0.25) (layer "B.Cu") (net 20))
 (segment (start 129.17 77.9925) (end 127.13 75.9525) (width 0.25) (layer "B.Cu") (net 20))
 (segment (start 135.67 91.5775) (end 129.17 85.0775) (width 0.25) (layer "B.Cu") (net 20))
 (segment (start 128.445 87.0525) (end 133.435 92.0425) (width 0.25) (layer "B.Cu") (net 14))
 (segment (start 139.3445 96.758) (end 139.83 96.2725) (width 0.25) (layer "B.Cu") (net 14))
 (segment (start 136.5505 96.758) (end 139.3445 96.758) (width 0.25) (layer "B.Cu") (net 14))
 (segment (start 133.435 92.0425) (end 133.435 93.3125) (width 0.25) (layer "B.Cu") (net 14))
 (segment (start 128.445 82.3475) (end 128.445 87.0525) (width 0.25) (layer "B.Cu") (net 14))
 (segment (start 133.435 93.3125) (end 133.27 93.4775) (width 0.25) (layer "B.Cu") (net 14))
 (segment (start 133.27 93.4775) (end 136.5505 96.758) (width 0.25) (layer "B.Cu") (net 14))
 (segment (start 127.13 81.0325) (end 128.445 82.3475) (width 0.25) (layer "B.Cu") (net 14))
 (segment (start 128.14 120.5975) (end 122.05 120.5975) (width 0.25) (layer "B.Cu") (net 7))
 (segment (start 132.205 116.5325) (end 128.14 120.5975) (width 0.25) (layer "B.Cu") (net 7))
 (segment (start 129.665 116.5325) (end 130.84 115.3575) (width 0.25) (layer "B.Cu") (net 8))
 (segment (start 135.957121 116.08292) (end 135.957121 123.064621) (width 0.25) (layer "B.Cu") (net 8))
 (segment (start 135.9 123.121743) (end 135.9 124.273257) (width 0.25) (layer "B.Cu") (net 8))
 (segment (start 135.231701 115.3575) (end 135.957121 116.08292) (width 0.25) (layer "B.Cu") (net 8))
 (segment (start 133.07 129.3775) (end 133.07 134.0075) (width 0.25) (layer "B.Cu") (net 8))
 (segment (start 133.07 134.0075) (end 137.29 138.2275) (width 0.25) (layer "B.Cu") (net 8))
 (segment (start 136.714243 125.0875) (end 136.714243 125.733257) (width 0.25) (layer "B.Cu") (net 8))
 (segment (start 135.9 124.273257) (end 136.714243 125.0875) (width 0.25) (layer "B.Cu") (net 8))
 (segment (start 136.714243 125.733257) (end 133.07 129.3775) (width 0.25) (layer "B.Cu") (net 8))
 (segment (start 130.84 115.3575) (end 135.231701 115.3575) (width 0.25) (layer "B.Cu") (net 8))
 (segment (start 135.957121 123.064621) (end 135.9 123.121743) (width 0.25) (layer "B.Cu") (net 8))
 (segment (start 135.14 147.4775) (end 124.2 147.4775) (width 0.25) (layer "B.Cu") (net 10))
 (segment (start 120.66 148.2375) (end 122.05 149.6275) (width 0.25) (layer "B.Cu") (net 10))
 (segment (start 123.585 116.5325) (end 124.585 116.5325) (width 0.25) (layer "B.Cu") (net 10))
 (segment (start 124.2 147.4775) (end 122.05 149.6275) (width 0.25) (layer "B.Cu") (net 10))
 (segment (start 139.07 147.8475) (end 137.29 149.6275) (width 0.25) (layer "B.Cu") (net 10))
 (segment (start 137.29 131.9975) (end 139.07 133.7775) (width 0.25) (layer "B.Cu") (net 10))
 (segment (start 137.29 149.6275) (end 135.14 147.4775) (width 0.25) (layer "B.Cu") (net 10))
 (segment (start 122.05 131.9975) (end 120.27 130.2175) (width 0.25) (layer "B.Cu") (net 10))
 (segment (start 120.27 130.2175) (end 120.27 119.8475) (width 0.25) (layer "B.Cu") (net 10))
 (segment (start 120.66 133.3875) (end 120.66 148.2375) (width 0.25) (layer "B.Cu") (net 10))
 (segment (start 139.07 133.7775) (end 139.07 147.8475) (width 0.25) (layer "B.Cu") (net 10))
 (segment (start 122.05 131.9975) (end 120.66 133.3875) (width 0.25) (layer "B.Cu") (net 10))
 (segment (start 120.27 119.8475) (end 123.585 116.5325) (width 0.25) (layer "B.Cu") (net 10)))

